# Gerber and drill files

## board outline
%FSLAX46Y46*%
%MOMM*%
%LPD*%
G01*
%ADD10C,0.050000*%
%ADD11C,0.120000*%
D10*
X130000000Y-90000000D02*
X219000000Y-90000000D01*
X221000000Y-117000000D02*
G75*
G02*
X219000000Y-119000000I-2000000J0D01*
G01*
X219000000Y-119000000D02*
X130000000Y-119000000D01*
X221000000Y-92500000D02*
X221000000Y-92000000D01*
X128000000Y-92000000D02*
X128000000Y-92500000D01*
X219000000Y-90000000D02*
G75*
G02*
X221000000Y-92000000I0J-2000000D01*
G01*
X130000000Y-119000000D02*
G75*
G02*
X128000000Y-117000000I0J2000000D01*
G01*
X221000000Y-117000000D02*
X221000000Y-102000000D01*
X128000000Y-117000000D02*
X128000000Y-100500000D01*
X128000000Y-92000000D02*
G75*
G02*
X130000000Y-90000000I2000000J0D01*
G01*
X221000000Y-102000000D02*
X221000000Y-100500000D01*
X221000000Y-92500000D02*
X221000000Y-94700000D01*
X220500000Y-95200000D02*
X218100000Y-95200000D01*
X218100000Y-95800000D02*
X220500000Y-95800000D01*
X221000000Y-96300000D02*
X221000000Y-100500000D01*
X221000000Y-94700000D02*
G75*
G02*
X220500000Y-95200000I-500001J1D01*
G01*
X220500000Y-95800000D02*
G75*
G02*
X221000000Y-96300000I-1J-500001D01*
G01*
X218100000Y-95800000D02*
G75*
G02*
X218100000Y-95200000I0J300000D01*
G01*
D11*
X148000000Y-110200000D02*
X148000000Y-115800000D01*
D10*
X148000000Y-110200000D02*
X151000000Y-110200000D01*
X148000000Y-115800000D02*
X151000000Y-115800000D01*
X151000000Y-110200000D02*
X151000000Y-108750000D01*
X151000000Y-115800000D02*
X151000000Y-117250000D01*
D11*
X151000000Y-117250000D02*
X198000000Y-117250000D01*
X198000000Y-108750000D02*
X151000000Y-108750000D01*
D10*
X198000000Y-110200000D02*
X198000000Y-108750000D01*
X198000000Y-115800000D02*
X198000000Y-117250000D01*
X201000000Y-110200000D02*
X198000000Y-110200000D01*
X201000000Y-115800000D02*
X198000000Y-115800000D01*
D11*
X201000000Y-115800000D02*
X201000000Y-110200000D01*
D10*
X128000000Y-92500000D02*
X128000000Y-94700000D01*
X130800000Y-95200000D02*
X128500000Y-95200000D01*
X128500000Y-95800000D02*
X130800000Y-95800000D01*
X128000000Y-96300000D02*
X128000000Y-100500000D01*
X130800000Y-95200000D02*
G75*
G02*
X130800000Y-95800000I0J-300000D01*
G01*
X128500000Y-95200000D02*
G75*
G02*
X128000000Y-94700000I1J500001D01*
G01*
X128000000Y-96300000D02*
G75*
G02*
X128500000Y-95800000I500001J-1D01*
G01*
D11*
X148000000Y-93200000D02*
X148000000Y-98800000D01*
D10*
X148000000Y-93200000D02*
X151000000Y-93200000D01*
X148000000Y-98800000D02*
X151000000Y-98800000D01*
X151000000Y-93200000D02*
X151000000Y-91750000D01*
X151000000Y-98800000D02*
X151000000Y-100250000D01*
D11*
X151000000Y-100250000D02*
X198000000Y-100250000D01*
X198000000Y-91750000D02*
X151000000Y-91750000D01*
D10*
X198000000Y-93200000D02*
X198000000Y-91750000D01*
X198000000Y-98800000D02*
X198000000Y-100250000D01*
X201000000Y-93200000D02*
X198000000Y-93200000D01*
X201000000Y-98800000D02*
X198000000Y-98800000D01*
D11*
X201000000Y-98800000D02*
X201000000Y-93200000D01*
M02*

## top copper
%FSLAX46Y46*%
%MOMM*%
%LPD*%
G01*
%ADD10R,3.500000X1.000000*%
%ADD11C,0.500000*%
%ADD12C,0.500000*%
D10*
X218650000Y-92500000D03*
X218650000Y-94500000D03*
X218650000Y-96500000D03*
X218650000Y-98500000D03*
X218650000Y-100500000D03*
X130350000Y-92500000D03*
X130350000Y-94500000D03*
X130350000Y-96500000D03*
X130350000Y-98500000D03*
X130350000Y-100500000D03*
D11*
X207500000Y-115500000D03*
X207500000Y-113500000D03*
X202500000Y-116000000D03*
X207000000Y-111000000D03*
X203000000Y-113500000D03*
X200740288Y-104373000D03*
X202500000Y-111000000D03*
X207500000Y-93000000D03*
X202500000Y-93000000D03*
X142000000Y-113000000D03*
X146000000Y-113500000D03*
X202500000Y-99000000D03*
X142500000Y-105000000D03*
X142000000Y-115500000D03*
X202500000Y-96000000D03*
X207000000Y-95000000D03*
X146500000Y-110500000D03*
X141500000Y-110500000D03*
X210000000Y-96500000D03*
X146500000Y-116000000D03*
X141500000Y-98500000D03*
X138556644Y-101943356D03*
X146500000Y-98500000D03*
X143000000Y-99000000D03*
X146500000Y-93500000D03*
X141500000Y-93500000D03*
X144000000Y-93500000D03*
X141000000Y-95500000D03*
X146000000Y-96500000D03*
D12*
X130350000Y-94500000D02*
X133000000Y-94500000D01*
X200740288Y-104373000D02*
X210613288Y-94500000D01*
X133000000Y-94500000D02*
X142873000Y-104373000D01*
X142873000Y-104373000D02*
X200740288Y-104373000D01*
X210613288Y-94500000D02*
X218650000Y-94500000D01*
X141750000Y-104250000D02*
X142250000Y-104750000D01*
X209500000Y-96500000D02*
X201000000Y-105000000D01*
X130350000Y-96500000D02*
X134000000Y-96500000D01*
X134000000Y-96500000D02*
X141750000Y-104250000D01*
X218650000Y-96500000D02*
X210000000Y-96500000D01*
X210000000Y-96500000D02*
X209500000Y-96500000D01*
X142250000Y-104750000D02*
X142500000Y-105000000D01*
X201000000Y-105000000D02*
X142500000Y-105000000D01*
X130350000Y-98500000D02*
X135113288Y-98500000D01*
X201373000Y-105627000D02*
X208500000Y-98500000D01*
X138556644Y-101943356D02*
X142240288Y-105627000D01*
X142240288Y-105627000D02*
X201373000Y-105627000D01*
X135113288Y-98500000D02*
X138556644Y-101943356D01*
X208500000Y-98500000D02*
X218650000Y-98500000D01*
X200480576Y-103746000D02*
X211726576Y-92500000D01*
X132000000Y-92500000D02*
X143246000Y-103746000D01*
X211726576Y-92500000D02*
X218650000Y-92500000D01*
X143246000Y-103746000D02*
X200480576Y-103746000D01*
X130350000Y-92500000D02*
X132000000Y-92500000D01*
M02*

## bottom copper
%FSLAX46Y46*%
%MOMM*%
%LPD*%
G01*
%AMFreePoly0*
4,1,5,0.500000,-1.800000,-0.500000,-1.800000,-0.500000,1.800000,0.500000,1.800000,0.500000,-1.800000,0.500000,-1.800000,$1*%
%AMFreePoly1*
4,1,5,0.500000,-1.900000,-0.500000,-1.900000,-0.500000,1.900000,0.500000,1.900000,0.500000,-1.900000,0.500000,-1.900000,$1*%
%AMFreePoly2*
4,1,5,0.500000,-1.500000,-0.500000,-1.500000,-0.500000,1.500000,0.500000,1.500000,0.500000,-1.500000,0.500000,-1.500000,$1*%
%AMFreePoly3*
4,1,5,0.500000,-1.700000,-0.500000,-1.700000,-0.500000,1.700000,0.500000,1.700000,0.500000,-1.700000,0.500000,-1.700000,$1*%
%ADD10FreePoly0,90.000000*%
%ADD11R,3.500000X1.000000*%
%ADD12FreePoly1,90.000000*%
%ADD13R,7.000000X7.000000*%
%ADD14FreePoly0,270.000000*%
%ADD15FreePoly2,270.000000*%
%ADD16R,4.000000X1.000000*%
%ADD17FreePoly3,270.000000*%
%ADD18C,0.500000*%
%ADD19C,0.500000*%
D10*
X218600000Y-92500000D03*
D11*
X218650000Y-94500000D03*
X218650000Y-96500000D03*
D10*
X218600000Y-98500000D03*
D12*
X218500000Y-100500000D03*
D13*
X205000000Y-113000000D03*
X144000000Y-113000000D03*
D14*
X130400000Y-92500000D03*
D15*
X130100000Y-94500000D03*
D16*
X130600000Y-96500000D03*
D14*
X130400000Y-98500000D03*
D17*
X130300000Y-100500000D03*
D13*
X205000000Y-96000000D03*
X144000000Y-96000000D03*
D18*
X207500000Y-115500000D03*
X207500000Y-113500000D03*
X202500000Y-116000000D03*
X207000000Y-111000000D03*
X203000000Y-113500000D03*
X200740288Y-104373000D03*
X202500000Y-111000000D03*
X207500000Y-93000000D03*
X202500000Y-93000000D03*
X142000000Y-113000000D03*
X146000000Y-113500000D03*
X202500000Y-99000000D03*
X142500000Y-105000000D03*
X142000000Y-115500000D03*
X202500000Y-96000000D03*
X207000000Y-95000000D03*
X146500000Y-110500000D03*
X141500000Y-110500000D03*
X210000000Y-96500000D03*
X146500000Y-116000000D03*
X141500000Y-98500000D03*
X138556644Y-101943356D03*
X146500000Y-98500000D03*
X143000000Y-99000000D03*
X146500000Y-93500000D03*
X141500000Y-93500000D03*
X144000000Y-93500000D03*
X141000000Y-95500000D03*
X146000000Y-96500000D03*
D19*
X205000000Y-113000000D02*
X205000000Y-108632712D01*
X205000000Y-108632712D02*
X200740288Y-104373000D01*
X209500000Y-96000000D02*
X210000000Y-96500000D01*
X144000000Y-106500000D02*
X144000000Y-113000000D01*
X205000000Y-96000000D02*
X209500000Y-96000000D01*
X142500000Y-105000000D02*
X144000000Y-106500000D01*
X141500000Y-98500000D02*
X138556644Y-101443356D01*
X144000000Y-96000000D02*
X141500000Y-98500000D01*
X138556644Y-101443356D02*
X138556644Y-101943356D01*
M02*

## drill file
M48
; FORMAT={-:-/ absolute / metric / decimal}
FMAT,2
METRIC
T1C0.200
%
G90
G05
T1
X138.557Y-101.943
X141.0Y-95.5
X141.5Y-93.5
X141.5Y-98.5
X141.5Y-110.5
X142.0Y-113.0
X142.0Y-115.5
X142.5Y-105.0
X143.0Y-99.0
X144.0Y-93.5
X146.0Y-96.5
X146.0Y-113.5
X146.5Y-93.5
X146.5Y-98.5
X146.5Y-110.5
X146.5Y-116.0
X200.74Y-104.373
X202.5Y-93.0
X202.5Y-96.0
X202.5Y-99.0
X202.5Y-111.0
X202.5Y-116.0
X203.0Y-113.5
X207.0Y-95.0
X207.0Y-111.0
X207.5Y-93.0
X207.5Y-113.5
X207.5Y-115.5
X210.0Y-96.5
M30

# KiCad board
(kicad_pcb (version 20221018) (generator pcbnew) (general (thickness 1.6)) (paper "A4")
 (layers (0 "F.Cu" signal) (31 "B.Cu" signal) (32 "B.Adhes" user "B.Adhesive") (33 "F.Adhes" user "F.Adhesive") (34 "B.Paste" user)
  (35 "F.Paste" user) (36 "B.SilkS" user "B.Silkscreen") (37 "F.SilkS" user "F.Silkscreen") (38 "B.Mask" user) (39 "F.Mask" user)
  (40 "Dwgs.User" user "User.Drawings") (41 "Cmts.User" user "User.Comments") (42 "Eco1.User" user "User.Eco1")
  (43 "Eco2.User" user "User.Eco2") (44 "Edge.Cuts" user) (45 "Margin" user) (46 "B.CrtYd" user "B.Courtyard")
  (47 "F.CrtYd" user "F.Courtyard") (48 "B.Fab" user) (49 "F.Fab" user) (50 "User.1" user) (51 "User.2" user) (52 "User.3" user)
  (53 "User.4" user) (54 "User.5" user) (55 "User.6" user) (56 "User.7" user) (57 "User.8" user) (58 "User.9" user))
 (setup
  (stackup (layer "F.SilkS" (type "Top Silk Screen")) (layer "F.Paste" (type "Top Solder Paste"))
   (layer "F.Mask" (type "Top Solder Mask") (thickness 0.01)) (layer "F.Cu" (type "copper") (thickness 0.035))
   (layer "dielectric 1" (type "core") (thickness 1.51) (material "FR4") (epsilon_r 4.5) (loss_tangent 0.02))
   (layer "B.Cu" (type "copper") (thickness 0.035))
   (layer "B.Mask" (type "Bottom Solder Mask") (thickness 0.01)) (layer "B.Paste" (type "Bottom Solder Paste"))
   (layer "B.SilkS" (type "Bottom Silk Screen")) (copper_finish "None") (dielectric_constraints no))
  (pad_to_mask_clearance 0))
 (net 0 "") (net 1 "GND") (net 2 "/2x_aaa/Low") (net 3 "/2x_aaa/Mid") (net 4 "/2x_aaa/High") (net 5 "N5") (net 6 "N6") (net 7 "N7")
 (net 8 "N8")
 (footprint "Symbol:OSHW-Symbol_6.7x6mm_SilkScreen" (layer "F.Cu") (at 185.25 104.5)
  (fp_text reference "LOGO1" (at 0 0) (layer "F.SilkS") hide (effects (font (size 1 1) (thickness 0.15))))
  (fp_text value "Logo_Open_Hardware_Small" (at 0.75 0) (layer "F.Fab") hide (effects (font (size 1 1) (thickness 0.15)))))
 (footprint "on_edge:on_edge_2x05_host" (layer "F.Cu") (at 221 96.5 -90)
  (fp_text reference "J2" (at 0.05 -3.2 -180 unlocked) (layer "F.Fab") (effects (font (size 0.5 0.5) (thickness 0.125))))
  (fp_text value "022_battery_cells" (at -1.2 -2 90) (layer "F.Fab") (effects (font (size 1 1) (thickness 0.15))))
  (fp_line (start -4 0) (end -1.8 0) (stroke (width 0.05) (type solid)) (layer "Edge.Cuts"))
  (fp_line (start -1.3 0.5) (end -1.3 2.9) (stroke (width 0.05) (type solid)) (layer "Edge.Cuts"))
  (fp_line (start -0.7 2.9) (end -0.7 0.5) (stroke (width 0.05) (type solid)) (layer "Edge.Cuts"))
  (fp_line (start -0.2 0) (end 4 0) (stroke (width 0.05) (type solid)) (layer "Edge.Cuts"))
  (fp_arc (start -1.8 0) (mid -1.446447 0.146447) (end -1.3 0.5) (stroke (width 0.05) (type solid)) (layer "Edge.Cuts"))
  (fp_arc (start -0.7 0.5) (mid -0.553553 0.146447) (end -0.2 0) (stroke (width 0.05) (type solid)) (layer "Edge.Cuts"))
  (fp_arc (start -0.7 2.9) (mid -1 3.2) (end -1.3 2.9) (stroke (width 0.05) (type solid)) (layer "Edge.Cuts"))
  (pad "1" smd rect (at -4 2.35 270) (size 1 3.5) (layers "F.Cu" "F.Mask") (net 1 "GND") (zone_connect 0))
  (pad "2" smd rect (at -2 2.35 270) (size 1 3.5) (layers "F.Cu" "F.Mask") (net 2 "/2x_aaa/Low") (zone_connect 0))
  (pad "3" smd rect (at 0 2.35 270) (size 1 3.5) (layers "F.Cu" "F.Mask") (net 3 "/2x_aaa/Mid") (zone_connect 0))
  (pad "4" smd rect (at 2 2.35 270) (size 1 3.5) (layers "F.Cu" "F.Mask") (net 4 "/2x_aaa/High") (zone_connect 0))
  (pad "5" smd rect (at 4 2.35 270) (size 1 3.5) (layers "F.Cu" "F.Mask") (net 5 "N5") (zone_connect 0))
  (pad "6" smd custom (at -4 2.4 90) (size 1 3.6) (layers "B.Cu" "B.Mask") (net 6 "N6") (zone_connect 0)
   (options (clearance outline) (anchor rect)) (primitives))
  (pad "7" smd rect (at -2 2.35 90) (size 1 3.5) (layers "B.Cu" "B.Mask") (zone_connect 0))
  (pad "8" smd rect (at 0 2.35 90) (size 1 3.5) (layers "B.Cu" "B.Mask") (zone_connect 0))
  (pad "9" smd custom (at 2 2.4 90) (size 1 3.6) (layers "B.Cu" "B.Mask") (zone_connect 0) (options (clearance outline) (anchor rect))
   (primitives))
  (pad "10" smd custom (at 4 2.5 90) (size 1 3.8) (layers "B.Cu" "B.Mask") (zone_connect 0) (options (clearance outline) (anchor rect))
   (primitives))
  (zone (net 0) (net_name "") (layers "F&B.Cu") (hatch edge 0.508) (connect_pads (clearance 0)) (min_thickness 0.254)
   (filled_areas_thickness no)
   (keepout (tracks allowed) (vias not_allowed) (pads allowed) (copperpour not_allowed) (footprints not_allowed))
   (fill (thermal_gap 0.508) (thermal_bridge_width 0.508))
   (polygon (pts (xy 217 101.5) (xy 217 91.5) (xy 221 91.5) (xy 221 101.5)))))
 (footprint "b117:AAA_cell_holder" (layer "F.Cu") (at 174.5 113)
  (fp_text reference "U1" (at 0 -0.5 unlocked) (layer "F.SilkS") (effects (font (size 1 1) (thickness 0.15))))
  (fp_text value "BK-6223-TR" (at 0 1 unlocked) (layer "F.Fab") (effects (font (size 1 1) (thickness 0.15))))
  (fp_line (start -26.5 -2.8) (end -26.5 2.8) (stroke (width 0.12) (type solid)) (layer "Edge.Cuts"))
  (fp_line (start -26.5 -2.8) (end -23.5 -2.8) (stroke (width 0.05) (type default)) (layer "Edge.Cuts"))
  (fp_line (start -26.5 2.8) (end -23.5 2.8) (stroke (width 0.05) (type default)) (layer "Edge.Cuts"))
  (fp_line (start -23.5 -2.8) (end -23.5 -4.25) (stroke (width 0.05) (type default)) (layer "Edge.Cuts"))
  (fp_line (start -23.5 2.8) (end -23.5 4.25) (stroke (width 0.05) (type default)) (layer "Edge.Cuts"))
  (fp_line (start -23.5 4.25) (end 23.5 4.25) (stroke (width 0.12) (type solid)) (layer "Edge.Cuts"))
  (fp_line (start 23.5 -4.25) (end -23.5 -4.25) (stroke (width 0.12) (type solid)) (layer "Edge.Cuts"))
  (fp_line (start 23.5 -2.8) (end 23.5 -4.25) (stroke (width 0.05) (type default)) (layer "Edge.Cuts"))
  (fp_line (start 23.5 2.8) (end 23.5 4.25) (stroke (width 0.05) (type default)) (layer "Edge.Cuts"))
  (fp_line (start 26.5 -2.8) (end 23.5 -2.8) (stroke (width 0.05) (type default)) (layer "Edge.Cuts"))
  (fp_line (start 26.5 2.8) (end 23.5 2.8) (stroke (width 0.05) (type default)) (layer "Edge.Cuts"))
  (fp_line (start 26.5 2.8) (end 26.5 -2.8) (stroke (width 0.12) (type solid)) (layer "Edge.Cuts"))
  (pad "1" smd rect (at 30.5 0) (size 7 7) (layers "B.Cu" "B.Paste" "B.Mask") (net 2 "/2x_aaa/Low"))
  (pad "2" smd rect (at -30.5 0) (size 7 7) (layers "B.Cu" "B.Paste" "B.Mask") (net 3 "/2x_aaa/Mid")))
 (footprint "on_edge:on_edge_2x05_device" (layer "F.Cu") (at 128 96.5 -90)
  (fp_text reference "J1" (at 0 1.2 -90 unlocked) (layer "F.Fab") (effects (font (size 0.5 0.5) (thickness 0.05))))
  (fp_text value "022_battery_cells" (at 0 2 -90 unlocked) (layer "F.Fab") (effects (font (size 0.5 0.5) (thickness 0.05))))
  (fp_line (start -4 0) (end -1.8 0) (stroke (width 0.05) (type solid)) (layer "Edge.Cuts"))
  (fp_line (start -1.3 -2.8) (end -1.3 -0.5) (stroke (width 0.05) (type solid)) (layer "Edge.Cuts"))
  (fp_line (start -0.7 -0.5) (end -0.7 -2.8) (stroke (width 0.05) (type solid)) (layer "Edge.Cuts"))
  (fp_line (start -0.2 0) (end 4 0) (stroke (width 0.05) (type solid)) (layer "Edge.Cuts"))
  (fp_arc (start -1.3 -2.8) (mid -1 -3.1) (end -0.7 -2.8) (stroke (width 0.05) (type solid)) (layer "Edge.Cuts"))
  (fp_arc (start -1.3 -0.5) (mid -1.446447 -0.146447) (end -1.8 0) (stroke (width 0.05) (type solid)) (layer "Edge.Cuts"))
  (fp_arc (start -0.2 0) (mid -0.553553 -0.146447) (end -0.7 -0.5) (stroke (width 0.05) (type solid)) (layer "Edge.Cuts"))
  (pad "1" smd rect (at -4 -2.35 90) (size 1 3.5) (layers "F.Cu" "F.Mask") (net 1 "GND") (zone_connect 0))
  (pad "2" smd rect (at -2 -2.35 270) (size 1 3.5) (layers "F.Cu" "F.Mask") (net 2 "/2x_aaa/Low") (zone_connect 0))
  (pad "3" smd rect (at 0 -2.35 270) (size 1 3.5) (layers "F.Cu" "F.Mask") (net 3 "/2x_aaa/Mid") (zone_connect 0))
  (pad "4" smd rect (at 2 -2.35 90) (size 1 3.5) (layers "F.Cu" "F.Mask") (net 4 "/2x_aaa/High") (zone_connect 0))
  (pad "5" smd rect (at 4 -2.35 90) (size 1 3.5) (layers "F.Cu" "F.Mask") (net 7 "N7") (zone_connect 0))
  (pad "6" smd custom (at -4 -2.4 270) (size 1 3.6) (layers "B.Cu" "B.Mask") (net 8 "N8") (zone_connect 0)
   (options (clearance outline) (anchor rect)) (primitives))
  (pad "7" smd custom (at -2 -2.1 270) (size 1 3) (layers "B.Cu" "B.Mask") (zone_connect 0) (options (clearance outline) (anchor rect))
   (primitives))
  (pad "8" smd rect (at 0 -2.6 270) (size 1 4) (layers "B.Cu" "B.Mask") (zone_connect 0))
  (pad "9" smd custom (at 2 -2.4 270) (size 1 3.6) (layers "B.Cu" "B.Mask") (zone_connect 0) (options (clearance outline) (anchor rect))
   (primitives))
  (pad "10" smd custom (at 4 -2.3 270) (size 1 3.4) (layers "B.Cu" "B.Mask") (zone_connect 0) (options (clearance outline) (anchor rect))
   (primitives))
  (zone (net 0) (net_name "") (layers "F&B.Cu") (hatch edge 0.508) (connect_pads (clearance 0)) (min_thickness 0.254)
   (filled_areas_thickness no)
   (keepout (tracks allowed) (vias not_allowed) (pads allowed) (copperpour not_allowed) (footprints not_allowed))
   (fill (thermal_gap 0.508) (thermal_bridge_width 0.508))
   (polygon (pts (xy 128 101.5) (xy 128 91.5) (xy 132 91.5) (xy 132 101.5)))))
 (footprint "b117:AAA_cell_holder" (layer "F.Cu") (at 174.5 96)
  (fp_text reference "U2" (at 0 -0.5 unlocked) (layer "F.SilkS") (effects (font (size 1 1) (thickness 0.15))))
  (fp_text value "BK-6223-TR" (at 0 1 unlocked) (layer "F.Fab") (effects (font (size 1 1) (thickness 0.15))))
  (fp_line (start -26.5 -2.8) (end -26.5 2.8) (stroke (width 0.12) (type solid)) (layer "Edge.Cuts"))
  (fp_line (start -26.5 -2.8) (end -23.5 -2.8) (stroke (width 0.05) (type default)) (layer "Edge.Cuts"))
  (fp_line (start -26.5 2.8) (end -23.5 2.8) (stroke (width 0.05) (type default)) (layer "Edge.Cuts"))
  (fp_line (start -23.5 -2.8) (end -23.5 -4.25) (stroke (width 0.05) (type default)) (layer "Edge.Cuts"))
  (fp_line (start -23.5 2.8) (end -23.5 4.25) (stroke (width 0.05) (type default)) (layer "Edge.Cuts"))
  (fp_line (start -23.5 4.25) (end 23.5 4.25) (stroke (width 0.12) (type solid)) (layer "Edge.Cuts"))
  (fp_line (start 23.5 -4.25) (end -23.5 -4.25) (stroke (width 0.12) (type solid)) (layer "Edge.Cuts"))
  (fp_line (start 23.5 -2.8) (end 23.5 -4.25) (stroke (width 0.05) (type default)) (layer "Edge.Cuts"))
  (fp_line (start 23.5 2.8) (end 23.5 4.25) (stroke (width 0.05) (type default)) (layer "Edge.Cuts"))
  (fp_line (start 26.5 -2.8) (end 23.5 -2.8) (stroke (width 0.05) (type default)) (layer "Edge.Cuts"))
  (fp_line (start 26.5 2.8) (end 23.5 2.8) (stroke (width 0.05) (type default)) (layer "Edge.Cuts"))
  (fp_line (start 26.5 2.8) (end 26.5 -2.8) (stroke (width 0.12) (type solid)) (layer "Edge.Cuts"))
  (pad "1" smd rect (at 30.5 0) (size 7 7) (layers "B.Cu" "B.Paste" "B.Mask") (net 3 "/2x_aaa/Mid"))
  (pad "2" smd rect (at -30.5 0) (size 7 7) (layers "B.Cu" "B.Paste" "B.Mask") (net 4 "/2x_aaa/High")))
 (gr_line (start 130 90) (end 219 90) (stroke (width 0.05) (type solid)) (layer "Edge.Cuts"))
 (gr_arc (start 221 117) (mid 220.414214 118.414214) (end 219 119) (stroke (width 0.05) (type solid)) (layer "Edge.Cuts"))
 (gr_line (start 219 119) (end 130 119) (stroke (width 0.05) (type solid)) (layer "Edge.Cuts"))
 (gr_line (start 221 92.5) (end 221 92) (stroke (width 0.05) (type solid)) (layer "Edge.Cuts"))
 (gr_line (start 128 92) (end 128 92.5) (stroke (width 0.05) (type solid)) (layer "Edge.Cuts"))
 (gr_arc (start 219 90) (mid 220.414214 90.585786) (end 221 92) (stroke (width 0.05) (type solid)) (layer "Edge.Cuts"))
 (gr_arc (start 130 119) (mid 128.585786 118.414214) (end 128 117) (stroke (width 0.05) (type solid)) (layer "Edge.Cuts"))
 (gr_line (start 221 117) (end 221 102) (stroke (width 0.05) (type solid)) (layer "Edge.Cuts"))
 (gr_line (start 128 117) (end 128 100.5) (stroke (width 0.05) (type solid)) (layer "Edge.Cuts"))
 (gr_arc (start 128 92) (mid 128.585786 90.585786) (end 130 90) (stroke (width 0.05) (type solid)) (layer "Edge.Cuts"))
 (gr_line (start 221 102) (end 221 100.5) (stroke (width 0.05) (type solid)) (layer "Edge.Cuts"))
 (segment (start 130.35 94.5) (end 133 94.5) (width 0.5) (layer "F.Cu") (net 2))
 (segment (start 200.740288 104.373) (end 210.613288 94.5) (width 0.5) (layer "F.Cu") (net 2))
 (segment (start 133 94.5) (end 142.873 104.373) (width 0.5) (layer "F.Cu") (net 2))
 (segment (start 142.873 104.373) (end 200.740288 104.373) (width 0.5) (layer "F.Cu") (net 2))
 (segment (start 210.613288 94.5) (end 218.65 94.5) (width 0.5) (layer "F.Cu") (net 2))
 (via (at 207.5 115.5) (size 0.5) (drill 0.2) (layers "F.Cu" "B.Cu") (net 2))
 (via (at 207.5 113.5) (size 0.5) (drill 0.2) (layers "F.Cu" "B.Cu") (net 2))
 (via (at 202.5 116) (size 0.5) (drill 0.2) (layers "F.Cu" "B.Cu") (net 2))
 (via (at 207 111) (size 0.5) (drill 0.2) (layers "F.Cu" "B.Cu") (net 2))
 (via (at 203 113.5) (size 0.5) (drill 0.2) (layers "F.Cu" "B.Cu") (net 2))
 (via (at 200.740288 104.373) (size 0.5) (drill 0.2) (layers "F.Cu" "B.Cu") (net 2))
 (via (at 202.5 111) (size 0.5) (drill 0.2) (layers "F.Cu" "B.Cu") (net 2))
 (segment (start 205 113) (end 205 108.632712) (width 0.5) (layer "B.Cu") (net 2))
 (segment (start 205 108.632712) (end 200.740288 104.373) (width 0.5) (layer "B.Cu") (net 2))
 (segment (start 141.75 104.25) (end 142.25 104.75) (width 0.5) (layer "F.Cu") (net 3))
 (segment (start 209.5 96.5) (end 201 105) (width 0.5) (layer "F.Cu") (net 3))
 (segment (start 130.35 96.5) (end 134 96.5) (width 0.5) (layer "F.Cu") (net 3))
 (segment (start 134 96.5) (end 141.75 104.25) (width 0.5) (layer "F.Cu") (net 3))
 (segment (start 218.65 96.5) (end 210 96.5) (width 0.5) (layer "F.Cu") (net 3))
 (segment (start 210 96.5) (end 209.5 96.5) (width 0.5) (layer "F.Cu") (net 3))
 (segment (start 142.25 104.75) (end 142.5 105) (width 0.5) (layer "F.Cu") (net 3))
 (segment (start 201 105) (end 142.5 105) (width 0.5) (layer "F.Cu") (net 3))
 (via (at 207.5 93) (size 0.5) (drill 0.2) (layers "F.Cu" "B.Cu") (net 3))
 (via (at 202.5 93) (size 0.5) (drill 0.2) (layers "F.Cu" "B.Cu") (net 3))
 (via (at 142 113) (size 0.5) (drill 0.2) (layers "F.Cu" "B.Cu") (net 3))
 (via (at 146 113.5) (size 0.5) (drill 0.2) (layers "F.Cu" "B.Cu") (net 3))
 (via (at 202.5 99) (size 0.5) (drill 0.2) (layers "F.Cu" "B.Cu") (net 3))
 (via (at 142.5 105) (size 0.5) (drill 0.2) (layers "F.Cu" "B.Cu") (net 3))
 (via (at 142 115.5) (size 0.5) (drill 0.2) (layers "F.Cu" "B.Cu") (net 3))
 (via (at 202.5 96) (size 0.5) (drill 0.2) (layers "F.Cu" "B.Cu") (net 3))
 (via (at 207 95) (size 0.5) (drill 0.2) (layers "F.Cu" "B.Cu") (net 3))
 (via (at 146.5 110.5) (size 0.5) (drill 0.2) (layers "F.Cu" "B.Cu") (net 3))
 (via (at 141.5 110.5) (size 0.5) (drill 0.2) (layers "F.Cu" "B.Cu") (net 3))
 (via (at 210 96.5) (size 0.5) (drill 0.2) (layers "F.Cu" "B.Cu") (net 3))
 (via (at 146.5 116) (size 0.5) (drill 0.2) (layers "F.Cu" "B.Cu") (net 3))
 (segment (start 209.5 96) (end 210 96.5) (width 0.5) (layer "B.Cu") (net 3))
 (segment (start 144 106.5) (end 144 113) (width 0.5) (layer "B.Cu") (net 3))
 (segment (start 205 96) (end 209.5 96) (width 0.5) (layer "B.Cu") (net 3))
 (segment (start 142.5 105) (end 144 106.5) (width 0.5) (layer "B.Cu") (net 3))
 (segment (start 130.35 98.5) (end 135.113288 98.5) (width 0.5) (layer "F.Cu") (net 4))
 (segment (start 201.373 105.627) (end 208.5 98.5) (width 0.5) (layer "F.Cu") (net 4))
 (segment (start 138.556644 101.943356) (end 142.240288 105.627) (width 0.5) (layer "F.Cu") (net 4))
 (segment (start 142.240288 105.627) (end 201.373 105.627) (width 0.5) (layer "F.Cu") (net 4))
 (segment (start 135.113288 98.5) (end 138.556644 101.943356) (width 0.5) (layer "F.Cu") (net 4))
 (segment (start 208.5 98.5) (end 218.65 98.5) (width 0.5) (layer "F.Cu") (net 4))
 (via (at 141.5 98.5) (size 0.5) (drill 0.2) (layers "F.Cu" "B.Cu") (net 4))
 (via (at 138.556644 101.943356) (size 0.5) (drill 0.2) (layers "F.Cu" "B.Cu") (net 4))
 (via (at 146.5 98.5) (size 0.5) (drill 0.2) (layers "F.Cu" "B.Cu") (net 4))
 (via (at 143 99) (size 0.5) (drill 0.2) (layers "F.Cu" "B.Cu") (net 4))
 (via (at 146.5 93.5) (size 0.5) (drill 0.2) (layers "F.Cu" "B.Cu") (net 4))
 (via (at 141.5 93.5) (size 0.5) (drill 0.2) (layers "F.Cu" "B.Cu") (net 4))
 (via (at 144 93.5) (size 0.5) (drill 0.2) (layers "F.Cu" "B.Cu") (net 4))
 (via (at 141 95.5) (size 0.5) (drill 0.2) (layers "F.Cu" "B.Cu") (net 4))
 (via (at 146 96.5) (size 0.5) (drill 0.2) (layers "F.Cu" "B.Cu") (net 4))
 (segment (start 141.5 98.5) (end 138.556644 101.443356) (width 0.5) (layer "B.Cu") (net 4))
 (segment (start 144 96) (end 141.5 98.5) (width 0.5) (layer "B.Cu") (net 4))
 (segment (start 138.556644 101.443356) (end 138.556644 101.943356) (width 0.5) (layer "B.Cu") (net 4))
 (segment (start 200.480576 103.746) (end 211.726576 92.5) (width 0.5) (layer "F.Cu") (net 1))
 (segment (start 132 92.5) (end 143.246 103.746) (width 0.5) (layer "F.Cu") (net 1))
 (segment (start 211.726576 92.5) (end 218.65 92.5) (width 0.5) (layer "F.Cu") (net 1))
 (segment (start 143.246 103.746) (end 200.480576 103.746) (width 0.5) (layer "F.Cu") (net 1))
 (segment (start 130.35 92.5) (end 132 92.5) (width 0.5) (layer "F.Cu") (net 1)))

